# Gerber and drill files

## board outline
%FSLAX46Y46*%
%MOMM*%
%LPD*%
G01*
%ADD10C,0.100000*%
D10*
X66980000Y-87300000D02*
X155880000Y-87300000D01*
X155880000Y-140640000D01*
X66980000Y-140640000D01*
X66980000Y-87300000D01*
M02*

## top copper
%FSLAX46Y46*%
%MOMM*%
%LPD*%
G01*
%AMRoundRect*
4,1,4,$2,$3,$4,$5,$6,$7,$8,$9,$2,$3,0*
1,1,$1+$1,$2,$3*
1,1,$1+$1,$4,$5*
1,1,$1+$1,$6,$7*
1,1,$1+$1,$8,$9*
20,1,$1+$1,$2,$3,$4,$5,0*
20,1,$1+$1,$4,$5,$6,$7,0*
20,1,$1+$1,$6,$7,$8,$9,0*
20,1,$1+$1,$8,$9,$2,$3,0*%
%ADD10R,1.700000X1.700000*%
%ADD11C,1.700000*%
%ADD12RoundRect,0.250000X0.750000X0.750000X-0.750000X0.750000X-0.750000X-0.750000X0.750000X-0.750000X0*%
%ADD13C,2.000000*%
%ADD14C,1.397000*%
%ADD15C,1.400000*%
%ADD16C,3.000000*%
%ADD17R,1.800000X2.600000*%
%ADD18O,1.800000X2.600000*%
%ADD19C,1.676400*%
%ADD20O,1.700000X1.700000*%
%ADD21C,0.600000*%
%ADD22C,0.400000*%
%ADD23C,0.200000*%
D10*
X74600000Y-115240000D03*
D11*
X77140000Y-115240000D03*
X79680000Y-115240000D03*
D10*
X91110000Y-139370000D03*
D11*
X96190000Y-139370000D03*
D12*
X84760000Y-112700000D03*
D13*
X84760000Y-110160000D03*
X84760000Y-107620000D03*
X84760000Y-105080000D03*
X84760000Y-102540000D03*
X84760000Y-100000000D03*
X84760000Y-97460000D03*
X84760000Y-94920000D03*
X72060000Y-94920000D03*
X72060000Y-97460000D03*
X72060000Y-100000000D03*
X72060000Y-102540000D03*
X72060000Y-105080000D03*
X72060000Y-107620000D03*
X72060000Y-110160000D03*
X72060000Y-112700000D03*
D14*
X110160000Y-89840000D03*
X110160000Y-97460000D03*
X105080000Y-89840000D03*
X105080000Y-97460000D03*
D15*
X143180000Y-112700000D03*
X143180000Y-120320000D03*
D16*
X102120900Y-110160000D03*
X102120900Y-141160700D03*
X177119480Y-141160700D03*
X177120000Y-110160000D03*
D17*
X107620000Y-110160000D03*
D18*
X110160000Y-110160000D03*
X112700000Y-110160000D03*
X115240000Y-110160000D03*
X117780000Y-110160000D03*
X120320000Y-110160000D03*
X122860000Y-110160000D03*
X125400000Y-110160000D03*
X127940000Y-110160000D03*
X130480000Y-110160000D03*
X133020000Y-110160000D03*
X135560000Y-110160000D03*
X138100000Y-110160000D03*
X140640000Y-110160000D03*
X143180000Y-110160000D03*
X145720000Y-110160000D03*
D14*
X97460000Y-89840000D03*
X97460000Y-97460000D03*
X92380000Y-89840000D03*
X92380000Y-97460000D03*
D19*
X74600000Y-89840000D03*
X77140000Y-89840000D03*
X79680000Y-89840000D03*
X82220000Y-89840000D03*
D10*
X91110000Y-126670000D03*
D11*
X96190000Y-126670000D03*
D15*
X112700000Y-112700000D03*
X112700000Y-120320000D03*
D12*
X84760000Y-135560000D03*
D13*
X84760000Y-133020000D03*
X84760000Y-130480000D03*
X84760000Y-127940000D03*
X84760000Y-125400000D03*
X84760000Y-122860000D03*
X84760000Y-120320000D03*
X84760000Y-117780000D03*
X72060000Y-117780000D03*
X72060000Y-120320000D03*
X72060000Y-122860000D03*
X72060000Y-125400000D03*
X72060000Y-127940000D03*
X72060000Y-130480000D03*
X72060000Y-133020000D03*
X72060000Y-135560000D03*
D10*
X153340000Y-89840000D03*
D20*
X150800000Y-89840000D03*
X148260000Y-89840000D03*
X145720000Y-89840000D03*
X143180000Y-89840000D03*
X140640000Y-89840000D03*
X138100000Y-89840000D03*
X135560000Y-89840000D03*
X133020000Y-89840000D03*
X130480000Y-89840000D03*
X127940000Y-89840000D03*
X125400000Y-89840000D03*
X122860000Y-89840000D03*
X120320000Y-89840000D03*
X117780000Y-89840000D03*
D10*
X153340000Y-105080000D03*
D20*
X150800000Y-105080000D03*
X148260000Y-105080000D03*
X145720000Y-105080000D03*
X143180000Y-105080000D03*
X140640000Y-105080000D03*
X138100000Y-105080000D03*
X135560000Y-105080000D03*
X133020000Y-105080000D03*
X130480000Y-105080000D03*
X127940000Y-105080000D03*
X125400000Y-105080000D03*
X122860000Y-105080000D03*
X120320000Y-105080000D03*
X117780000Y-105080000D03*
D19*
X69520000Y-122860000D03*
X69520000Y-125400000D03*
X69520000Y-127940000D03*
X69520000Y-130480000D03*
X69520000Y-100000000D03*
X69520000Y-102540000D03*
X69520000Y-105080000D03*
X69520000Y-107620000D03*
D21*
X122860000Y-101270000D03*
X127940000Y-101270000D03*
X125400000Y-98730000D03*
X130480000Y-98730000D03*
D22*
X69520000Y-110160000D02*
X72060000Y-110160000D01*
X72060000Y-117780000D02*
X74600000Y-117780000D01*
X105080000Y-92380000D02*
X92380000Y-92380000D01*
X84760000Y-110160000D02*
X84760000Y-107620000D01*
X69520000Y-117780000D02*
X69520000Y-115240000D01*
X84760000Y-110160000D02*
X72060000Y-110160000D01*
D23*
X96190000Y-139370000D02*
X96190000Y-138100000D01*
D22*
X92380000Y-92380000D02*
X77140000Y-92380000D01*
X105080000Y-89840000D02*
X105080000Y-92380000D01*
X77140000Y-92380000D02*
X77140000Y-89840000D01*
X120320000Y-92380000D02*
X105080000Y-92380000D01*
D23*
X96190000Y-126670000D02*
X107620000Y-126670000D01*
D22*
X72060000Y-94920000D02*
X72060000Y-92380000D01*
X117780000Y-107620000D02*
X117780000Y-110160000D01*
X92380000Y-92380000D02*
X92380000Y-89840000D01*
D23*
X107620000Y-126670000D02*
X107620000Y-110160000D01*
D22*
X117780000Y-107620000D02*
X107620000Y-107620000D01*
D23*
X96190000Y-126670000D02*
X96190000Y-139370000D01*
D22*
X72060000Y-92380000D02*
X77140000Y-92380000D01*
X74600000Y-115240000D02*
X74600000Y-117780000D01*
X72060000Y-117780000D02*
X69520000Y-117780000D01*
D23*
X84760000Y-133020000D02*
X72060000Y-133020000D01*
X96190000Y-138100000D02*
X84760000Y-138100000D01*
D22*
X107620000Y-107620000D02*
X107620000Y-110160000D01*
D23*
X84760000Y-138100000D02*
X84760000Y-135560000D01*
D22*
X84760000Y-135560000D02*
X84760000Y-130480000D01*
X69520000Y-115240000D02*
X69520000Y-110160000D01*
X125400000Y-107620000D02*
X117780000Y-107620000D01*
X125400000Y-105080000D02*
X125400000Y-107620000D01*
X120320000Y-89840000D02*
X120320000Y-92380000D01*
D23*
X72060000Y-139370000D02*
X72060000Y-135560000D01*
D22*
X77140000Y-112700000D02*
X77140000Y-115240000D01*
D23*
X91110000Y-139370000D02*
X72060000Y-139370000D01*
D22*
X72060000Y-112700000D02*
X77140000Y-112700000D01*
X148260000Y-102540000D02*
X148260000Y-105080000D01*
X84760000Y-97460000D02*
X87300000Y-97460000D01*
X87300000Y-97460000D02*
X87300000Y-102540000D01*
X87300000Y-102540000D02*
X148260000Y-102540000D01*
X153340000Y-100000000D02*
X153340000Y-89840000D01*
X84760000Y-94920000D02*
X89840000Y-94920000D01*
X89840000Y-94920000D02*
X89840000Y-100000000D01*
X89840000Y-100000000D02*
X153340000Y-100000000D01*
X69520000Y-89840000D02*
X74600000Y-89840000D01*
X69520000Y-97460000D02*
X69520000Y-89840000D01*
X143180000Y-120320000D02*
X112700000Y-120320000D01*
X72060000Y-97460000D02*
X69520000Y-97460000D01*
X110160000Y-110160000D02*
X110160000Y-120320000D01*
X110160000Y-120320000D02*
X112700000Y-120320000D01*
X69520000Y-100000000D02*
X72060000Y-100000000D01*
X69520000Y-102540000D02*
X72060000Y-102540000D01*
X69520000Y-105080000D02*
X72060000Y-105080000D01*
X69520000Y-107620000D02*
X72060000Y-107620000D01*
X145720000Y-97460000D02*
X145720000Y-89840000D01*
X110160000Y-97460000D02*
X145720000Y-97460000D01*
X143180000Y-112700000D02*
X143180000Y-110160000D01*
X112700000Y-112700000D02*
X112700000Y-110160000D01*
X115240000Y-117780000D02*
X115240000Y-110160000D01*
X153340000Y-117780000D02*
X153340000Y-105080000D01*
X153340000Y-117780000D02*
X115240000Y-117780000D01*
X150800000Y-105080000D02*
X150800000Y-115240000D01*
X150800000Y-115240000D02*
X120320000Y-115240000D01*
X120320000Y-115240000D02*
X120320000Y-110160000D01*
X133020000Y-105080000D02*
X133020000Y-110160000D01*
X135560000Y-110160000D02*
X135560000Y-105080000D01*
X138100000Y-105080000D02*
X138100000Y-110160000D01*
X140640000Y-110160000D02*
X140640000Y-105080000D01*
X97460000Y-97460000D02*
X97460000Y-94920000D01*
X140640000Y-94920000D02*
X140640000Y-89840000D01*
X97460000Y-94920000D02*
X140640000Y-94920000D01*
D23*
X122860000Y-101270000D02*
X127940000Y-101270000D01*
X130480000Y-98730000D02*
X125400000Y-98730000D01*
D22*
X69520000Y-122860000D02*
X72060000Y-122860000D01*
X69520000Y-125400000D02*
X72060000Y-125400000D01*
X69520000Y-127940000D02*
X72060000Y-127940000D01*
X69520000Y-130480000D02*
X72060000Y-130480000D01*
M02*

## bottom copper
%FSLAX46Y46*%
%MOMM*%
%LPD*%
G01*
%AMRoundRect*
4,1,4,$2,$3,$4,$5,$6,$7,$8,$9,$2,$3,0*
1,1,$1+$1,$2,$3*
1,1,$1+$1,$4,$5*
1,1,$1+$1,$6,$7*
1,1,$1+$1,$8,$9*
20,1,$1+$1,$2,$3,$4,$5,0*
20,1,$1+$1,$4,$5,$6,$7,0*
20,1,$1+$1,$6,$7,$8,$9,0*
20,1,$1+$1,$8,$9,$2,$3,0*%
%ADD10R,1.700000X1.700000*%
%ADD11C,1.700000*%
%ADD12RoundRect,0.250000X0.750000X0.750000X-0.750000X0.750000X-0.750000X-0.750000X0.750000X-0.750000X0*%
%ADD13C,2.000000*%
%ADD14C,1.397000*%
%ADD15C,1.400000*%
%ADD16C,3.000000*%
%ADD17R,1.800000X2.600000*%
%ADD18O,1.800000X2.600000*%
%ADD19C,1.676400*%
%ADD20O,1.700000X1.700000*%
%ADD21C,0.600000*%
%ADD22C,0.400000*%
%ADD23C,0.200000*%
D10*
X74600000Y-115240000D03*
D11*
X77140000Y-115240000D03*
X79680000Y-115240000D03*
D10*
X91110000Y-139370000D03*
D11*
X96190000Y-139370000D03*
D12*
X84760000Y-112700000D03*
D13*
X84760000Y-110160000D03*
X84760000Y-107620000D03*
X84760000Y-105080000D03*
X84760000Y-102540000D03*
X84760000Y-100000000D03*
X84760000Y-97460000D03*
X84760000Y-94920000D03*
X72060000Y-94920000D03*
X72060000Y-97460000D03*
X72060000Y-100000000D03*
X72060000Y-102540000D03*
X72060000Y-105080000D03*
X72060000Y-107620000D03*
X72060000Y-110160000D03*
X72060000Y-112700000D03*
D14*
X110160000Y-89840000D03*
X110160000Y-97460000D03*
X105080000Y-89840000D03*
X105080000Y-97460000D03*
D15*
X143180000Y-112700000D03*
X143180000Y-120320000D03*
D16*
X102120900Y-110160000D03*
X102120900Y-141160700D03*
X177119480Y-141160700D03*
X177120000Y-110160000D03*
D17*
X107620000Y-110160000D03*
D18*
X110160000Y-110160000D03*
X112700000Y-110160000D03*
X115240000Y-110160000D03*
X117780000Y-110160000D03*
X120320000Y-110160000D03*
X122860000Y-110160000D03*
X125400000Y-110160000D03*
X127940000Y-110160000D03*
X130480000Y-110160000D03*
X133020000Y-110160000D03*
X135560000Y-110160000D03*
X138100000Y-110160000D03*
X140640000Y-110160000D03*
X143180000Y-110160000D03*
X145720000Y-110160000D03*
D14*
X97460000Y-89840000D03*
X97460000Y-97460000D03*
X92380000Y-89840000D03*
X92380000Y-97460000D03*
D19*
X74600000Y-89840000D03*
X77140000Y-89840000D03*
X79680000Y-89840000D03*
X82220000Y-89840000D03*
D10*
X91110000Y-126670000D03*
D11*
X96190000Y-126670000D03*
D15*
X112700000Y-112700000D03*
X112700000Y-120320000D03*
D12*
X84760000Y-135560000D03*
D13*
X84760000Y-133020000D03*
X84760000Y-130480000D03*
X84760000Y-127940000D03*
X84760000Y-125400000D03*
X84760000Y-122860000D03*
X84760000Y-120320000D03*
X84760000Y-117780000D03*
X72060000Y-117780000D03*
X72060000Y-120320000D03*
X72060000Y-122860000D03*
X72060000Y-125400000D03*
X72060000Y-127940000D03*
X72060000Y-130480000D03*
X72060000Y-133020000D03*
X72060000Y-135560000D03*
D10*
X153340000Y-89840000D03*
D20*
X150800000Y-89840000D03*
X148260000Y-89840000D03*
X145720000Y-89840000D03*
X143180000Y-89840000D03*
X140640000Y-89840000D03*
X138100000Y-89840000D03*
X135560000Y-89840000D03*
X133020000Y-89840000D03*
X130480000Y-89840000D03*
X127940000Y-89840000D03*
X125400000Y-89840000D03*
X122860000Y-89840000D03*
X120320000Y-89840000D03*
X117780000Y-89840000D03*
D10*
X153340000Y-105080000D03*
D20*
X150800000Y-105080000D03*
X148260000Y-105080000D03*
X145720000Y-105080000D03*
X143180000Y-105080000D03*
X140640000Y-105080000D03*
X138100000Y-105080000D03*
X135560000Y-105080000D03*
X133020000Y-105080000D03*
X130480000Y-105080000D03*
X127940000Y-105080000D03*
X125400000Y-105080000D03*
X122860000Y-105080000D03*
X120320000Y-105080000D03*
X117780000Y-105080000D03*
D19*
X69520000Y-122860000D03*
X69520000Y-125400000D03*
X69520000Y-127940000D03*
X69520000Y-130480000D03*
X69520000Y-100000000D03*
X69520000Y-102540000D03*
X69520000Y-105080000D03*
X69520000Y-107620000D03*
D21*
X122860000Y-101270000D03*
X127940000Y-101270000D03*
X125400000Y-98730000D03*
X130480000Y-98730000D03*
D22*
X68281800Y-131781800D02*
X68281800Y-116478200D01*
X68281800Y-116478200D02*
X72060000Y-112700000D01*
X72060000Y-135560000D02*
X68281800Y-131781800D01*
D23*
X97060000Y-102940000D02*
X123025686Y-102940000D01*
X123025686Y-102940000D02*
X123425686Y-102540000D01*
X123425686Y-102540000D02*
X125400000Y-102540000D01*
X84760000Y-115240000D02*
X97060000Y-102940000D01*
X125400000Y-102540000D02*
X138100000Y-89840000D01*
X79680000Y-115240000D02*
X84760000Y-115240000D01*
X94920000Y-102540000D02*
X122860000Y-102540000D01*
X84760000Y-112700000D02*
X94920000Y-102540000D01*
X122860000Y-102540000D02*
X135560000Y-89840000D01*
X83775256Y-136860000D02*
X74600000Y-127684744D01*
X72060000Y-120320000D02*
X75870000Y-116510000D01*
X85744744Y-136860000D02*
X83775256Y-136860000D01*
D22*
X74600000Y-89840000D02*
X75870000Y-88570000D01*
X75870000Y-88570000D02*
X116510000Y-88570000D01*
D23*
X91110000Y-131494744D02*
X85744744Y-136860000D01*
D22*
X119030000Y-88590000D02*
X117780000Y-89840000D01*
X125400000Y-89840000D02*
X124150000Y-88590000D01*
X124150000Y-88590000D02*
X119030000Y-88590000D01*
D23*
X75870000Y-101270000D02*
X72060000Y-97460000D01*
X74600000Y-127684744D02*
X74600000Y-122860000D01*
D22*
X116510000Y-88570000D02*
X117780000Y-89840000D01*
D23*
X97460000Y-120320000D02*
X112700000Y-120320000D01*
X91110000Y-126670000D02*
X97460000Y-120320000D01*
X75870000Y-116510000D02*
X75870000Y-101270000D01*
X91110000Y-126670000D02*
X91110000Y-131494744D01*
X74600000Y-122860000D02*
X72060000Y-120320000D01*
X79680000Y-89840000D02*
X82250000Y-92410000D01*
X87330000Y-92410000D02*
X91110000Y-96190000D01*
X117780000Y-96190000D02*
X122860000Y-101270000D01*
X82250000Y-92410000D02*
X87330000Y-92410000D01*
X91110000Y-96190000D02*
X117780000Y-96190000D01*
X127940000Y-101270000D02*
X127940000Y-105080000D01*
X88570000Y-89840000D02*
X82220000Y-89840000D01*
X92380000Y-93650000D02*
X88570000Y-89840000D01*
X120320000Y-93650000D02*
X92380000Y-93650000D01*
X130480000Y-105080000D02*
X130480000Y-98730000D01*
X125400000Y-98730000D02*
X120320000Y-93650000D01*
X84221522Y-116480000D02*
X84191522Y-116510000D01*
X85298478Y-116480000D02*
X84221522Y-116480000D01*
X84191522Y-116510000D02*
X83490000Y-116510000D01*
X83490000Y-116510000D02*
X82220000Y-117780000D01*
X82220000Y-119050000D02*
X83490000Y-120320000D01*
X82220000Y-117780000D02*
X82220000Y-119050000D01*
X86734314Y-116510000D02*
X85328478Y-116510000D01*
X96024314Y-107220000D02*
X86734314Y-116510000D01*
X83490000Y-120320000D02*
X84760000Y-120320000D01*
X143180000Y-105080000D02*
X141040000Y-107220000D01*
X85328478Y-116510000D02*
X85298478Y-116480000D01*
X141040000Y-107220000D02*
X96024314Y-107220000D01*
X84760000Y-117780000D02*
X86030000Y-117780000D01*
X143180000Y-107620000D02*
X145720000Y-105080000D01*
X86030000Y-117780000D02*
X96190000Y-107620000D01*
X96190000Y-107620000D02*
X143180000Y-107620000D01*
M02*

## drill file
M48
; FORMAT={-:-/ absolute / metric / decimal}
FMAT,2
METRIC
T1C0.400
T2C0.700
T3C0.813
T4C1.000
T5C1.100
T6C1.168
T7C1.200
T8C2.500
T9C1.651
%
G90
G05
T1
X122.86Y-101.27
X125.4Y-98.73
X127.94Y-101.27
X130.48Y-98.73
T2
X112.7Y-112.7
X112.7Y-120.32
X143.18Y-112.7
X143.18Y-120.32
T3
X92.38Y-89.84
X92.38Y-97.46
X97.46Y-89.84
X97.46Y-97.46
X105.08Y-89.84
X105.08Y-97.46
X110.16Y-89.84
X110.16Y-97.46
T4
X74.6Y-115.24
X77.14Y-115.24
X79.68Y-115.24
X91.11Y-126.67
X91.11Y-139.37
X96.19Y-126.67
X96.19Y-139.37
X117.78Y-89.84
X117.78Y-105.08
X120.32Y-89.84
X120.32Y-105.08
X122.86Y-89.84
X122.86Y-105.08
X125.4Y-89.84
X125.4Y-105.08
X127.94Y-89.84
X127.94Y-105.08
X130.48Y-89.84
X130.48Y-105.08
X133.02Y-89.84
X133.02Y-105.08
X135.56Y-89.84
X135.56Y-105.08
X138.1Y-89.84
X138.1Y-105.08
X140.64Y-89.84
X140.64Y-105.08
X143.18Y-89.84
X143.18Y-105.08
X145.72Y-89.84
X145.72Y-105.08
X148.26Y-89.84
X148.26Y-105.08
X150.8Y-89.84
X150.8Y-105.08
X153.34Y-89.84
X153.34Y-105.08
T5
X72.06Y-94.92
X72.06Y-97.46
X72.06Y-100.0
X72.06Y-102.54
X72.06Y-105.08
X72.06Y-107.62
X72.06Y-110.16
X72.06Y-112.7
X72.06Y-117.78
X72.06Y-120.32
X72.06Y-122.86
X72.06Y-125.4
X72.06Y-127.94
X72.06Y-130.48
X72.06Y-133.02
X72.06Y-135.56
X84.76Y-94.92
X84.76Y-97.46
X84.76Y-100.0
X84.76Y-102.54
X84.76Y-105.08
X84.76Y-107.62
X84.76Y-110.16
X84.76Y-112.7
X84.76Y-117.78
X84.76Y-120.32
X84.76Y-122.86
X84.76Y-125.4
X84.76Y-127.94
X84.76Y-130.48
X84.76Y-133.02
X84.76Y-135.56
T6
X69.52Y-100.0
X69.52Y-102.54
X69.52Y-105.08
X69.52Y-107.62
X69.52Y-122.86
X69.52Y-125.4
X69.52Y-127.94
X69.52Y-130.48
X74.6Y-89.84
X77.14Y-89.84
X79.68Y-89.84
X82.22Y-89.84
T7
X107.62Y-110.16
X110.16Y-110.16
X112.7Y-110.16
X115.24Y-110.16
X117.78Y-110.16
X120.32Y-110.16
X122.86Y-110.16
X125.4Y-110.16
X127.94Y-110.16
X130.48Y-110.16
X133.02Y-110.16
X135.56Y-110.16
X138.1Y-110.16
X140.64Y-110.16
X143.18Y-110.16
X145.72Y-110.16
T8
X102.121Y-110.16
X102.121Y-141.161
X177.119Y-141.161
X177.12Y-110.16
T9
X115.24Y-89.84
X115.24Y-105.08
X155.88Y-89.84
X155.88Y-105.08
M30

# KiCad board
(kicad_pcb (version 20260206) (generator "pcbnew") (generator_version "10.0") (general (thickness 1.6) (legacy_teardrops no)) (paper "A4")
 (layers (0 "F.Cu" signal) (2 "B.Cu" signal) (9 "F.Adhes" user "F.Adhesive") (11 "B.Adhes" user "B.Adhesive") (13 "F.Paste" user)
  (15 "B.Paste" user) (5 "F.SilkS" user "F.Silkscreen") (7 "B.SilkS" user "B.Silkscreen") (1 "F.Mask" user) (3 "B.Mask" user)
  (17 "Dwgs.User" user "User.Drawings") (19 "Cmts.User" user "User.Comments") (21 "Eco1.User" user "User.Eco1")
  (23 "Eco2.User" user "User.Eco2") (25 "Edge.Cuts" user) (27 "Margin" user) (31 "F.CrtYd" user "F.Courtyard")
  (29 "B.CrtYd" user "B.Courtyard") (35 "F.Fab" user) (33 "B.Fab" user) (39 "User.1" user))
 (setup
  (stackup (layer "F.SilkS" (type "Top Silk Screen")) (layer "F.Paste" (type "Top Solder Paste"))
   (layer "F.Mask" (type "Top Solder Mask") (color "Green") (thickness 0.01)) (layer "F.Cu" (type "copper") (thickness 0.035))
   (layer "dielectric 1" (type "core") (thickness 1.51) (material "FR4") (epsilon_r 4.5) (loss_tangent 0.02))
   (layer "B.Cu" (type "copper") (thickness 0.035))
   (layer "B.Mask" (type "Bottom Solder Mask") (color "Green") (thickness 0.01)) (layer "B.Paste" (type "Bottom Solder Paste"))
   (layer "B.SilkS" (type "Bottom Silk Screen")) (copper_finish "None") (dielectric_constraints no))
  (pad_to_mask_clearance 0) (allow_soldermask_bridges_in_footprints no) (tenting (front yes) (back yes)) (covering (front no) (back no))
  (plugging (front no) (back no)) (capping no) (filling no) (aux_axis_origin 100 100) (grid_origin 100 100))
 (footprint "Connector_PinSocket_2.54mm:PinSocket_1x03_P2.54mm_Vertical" (layer "F.Cu") (at 74.6 115.24 90)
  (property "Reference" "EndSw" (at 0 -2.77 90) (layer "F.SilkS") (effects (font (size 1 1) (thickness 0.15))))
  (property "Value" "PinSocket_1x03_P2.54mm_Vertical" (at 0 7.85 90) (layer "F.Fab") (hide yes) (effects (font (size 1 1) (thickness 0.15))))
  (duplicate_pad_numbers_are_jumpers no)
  (pad "1" thru_hole rect (at 0 0 90) (size 1.7 1.7) (drill 1) (layers "*.Cu" "*.Mask") (remove_unused_layers no) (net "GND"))
  (pad "2" thru_hole circle (at 0 2.54 90) (size 1.7 1.7) (drill 1) (layers "*.Cu" "*.Mask") (remove_unused_layers no) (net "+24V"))
  (pad "3" thru_hole circle (at 0 5.08 90) (size 1.7 1.7) (drill 1) (layers "*.Cu" "*.Mask") (remove_unused_layers no) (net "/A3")))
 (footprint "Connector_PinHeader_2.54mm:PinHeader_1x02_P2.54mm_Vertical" (layer "F.Cu") (at 91.11 139.37 90)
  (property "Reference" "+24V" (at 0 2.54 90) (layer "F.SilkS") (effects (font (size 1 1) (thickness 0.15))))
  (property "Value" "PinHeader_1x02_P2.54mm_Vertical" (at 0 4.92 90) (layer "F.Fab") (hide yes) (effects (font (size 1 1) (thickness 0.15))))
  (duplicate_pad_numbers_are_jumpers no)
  (pad "1" thru_hole rect (at 0 0 90) (size 1.7 1.7) (drill 1) (layers "*.Cu" "*.Mask") (remove_unused_layers no) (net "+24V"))
  (pad "2" thru_hole circle (at 0 5.08 90) (size 1.7 1.7) (drill 1) (layers "*.Cu" "*.Mask") (remove_unused_layers no) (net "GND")))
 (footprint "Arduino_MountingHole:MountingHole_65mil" (layer "F.Cu") (at 155.88 105.08 180)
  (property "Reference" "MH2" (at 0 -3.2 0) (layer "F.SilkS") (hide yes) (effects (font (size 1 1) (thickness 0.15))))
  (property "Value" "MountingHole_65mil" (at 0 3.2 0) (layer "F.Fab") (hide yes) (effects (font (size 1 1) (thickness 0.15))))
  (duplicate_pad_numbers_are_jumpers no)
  (pad "" np_thru_hole circle (at 0 0 180) (size 1.651 1.651) (drill 1.651) (layers "*.Cu" "*.Mask")))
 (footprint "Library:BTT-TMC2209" (layer "F.Cu") (at 86.03 113.97 180)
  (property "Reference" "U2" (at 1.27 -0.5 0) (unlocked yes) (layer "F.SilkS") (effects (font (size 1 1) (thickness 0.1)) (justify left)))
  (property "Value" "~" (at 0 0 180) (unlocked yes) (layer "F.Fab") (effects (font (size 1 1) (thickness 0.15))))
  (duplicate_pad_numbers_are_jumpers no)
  (pad "1" thru_hole roundrect (at 1.27 1.27 180) (size 2 2) (drill 1.1) (layers "*.Cu" "*.Mask") (remove_unused_layers no)
   (roundrect_rratio 0.125) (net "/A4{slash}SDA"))
  (pad "2" thru_hole circle (at 1.27 3.81 180) (size 2 2) (drill 1.1) (layers "*.Cu" "*.Mask") (remove_unused_layers no) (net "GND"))
  (pad "3" thru_hole circle (at 1.27 6.35 180) (size 2 2) (drill 1.1) (layers "*.Cu" "*.Mask") (remove_unused_layers no) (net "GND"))
  (pad "4" thru_hole circle (at 1.27 8.89 180) (size 2 2) (drill 1.1) (layers "*.Cu" "*.Mask") (remove_unused_layers no)
   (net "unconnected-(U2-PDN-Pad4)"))
  (pad "5" thru_hole circle (at 1.27 11.43 180) (size 2 2) (drill 1.1) (layers "*.Cu" "*.Mask") (remove_unused_layers no)
   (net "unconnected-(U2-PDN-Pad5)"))
  (pad "6" thru_hole circle (at 1.27 13.97 180) (size 2 2) (drill 1.1) (layers "*.Cu" "*.Mask") (remove_unused_layers no)
   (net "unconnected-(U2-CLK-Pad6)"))
  (pad "7" thru_hole circle (at 1.27 16.51 180) (size 2 2) (drill 1.1) (layers "*.Cu" "*.Mask") (remove_unused_layers no)
   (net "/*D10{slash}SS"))
  (pad "8" thru_hole circle (at 1.27 19.05 180) (size 2 2) (drill 1.1) (layers "*.Cu" "*.Mask") (remove_unused_layers no)
   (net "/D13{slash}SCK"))
  (pad "9" thru_hole circle (at 13.97 19.05 180) (size 2 2) (drill 1.1) (layers "*.Cu" "*.Mask") (remove_unused_layers no) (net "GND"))
  (pad "10" thru_hole circle (at 13.97 16.51 180) (size 2 2) (drill 1.1) (layers "*.Cu" "*.Mask") (remove_unused_layers no) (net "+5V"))
  (pad "11" thru_hole circle (at 13.97 13.97 180) (size 2 2) (drill 1.1) (layers "*.Cu" "*.Mask") (remove_unused_layers no)
   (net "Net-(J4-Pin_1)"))
  (pad "12" thru_hole circle (at 13.97 11.43 180) (size 2 2) (drill 1.1) (layers "*.Cu" "*.Mask") (remove_unused_layers no)
   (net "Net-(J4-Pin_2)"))
  (pad "13" thru_hole circle (at 13.97 8.89 180) (size 2 2) (drill 1.1) (layers "*.Cu" "*.Mask") (remove_unused_layers no)
   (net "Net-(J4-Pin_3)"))
  (pad "14" thru_hole circle (at 13.97 6.35 180) (size 2 2) (drill 1.1) (layers "*.Cu" "*.Mask") (remove_unused_layers no)
   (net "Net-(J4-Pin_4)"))
  (pad "15" thru_hole circle (at 13.97 3.81 180) (size 2 2) (drill 1.1) (layers "*.Cu" "*.Mask") (remove_unused_layers no) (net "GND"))
  (pad "16" thru_hole circle (at 13.97 1.27 180) (size 2 2) (drill 1.1) (layers "*.Cu" "*.Mask") (remove_unused_layers no) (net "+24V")))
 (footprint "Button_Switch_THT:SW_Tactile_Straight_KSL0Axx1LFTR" (layer "F.Cu") (at 110.16 89.84 -90)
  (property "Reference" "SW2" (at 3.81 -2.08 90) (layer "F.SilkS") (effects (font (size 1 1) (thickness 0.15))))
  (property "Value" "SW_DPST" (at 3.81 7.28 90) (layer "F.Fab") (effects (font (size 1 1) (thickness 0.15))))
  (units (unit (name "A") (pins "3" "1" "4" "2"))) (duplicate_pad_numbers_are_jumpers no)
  (pad "1" thru_hole circle (at 0 0 270) (size 1.397 1.397) (drill 0.8128) (layers "*.Cu" "*.Mask") (remove_unused_layers no))
  (pad "1" thru_hole circle (at 7.62 0 270) (size 1.397 1.397) (drill 0.8128) (layers "*.Cu" "*.Mask") (remove_unused_layers no) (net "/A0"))
  (pad "2" thru_hole circle (at 0 5.08 270) (size 1.397 1.397) (drill 0.8128) (layers "*.Cu" "*.Mask") (remove_unused_layers no) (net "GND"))
  (pad "2" thru_hole circle (at 7.62 5.08 270) (size 1.397 1.397) (drill 0.8128) (layers "*.Cu" "*.Mask") (remove_unused_layers no)))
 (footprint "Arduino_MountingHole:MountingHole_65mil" (layer "F.Cu") (at 115.24 89.84 180)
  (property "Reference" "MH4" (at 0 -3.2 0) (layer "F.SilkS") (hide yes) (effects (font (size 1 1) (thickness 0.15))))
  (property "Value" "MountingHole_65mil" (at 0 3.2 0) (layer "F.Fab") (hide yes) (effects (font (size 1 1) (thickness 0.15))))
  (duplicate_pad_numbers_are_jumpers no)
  (pad "" np_thru_hole circle (at 0 0 180) (size 1.651 1.651) (drill 1.651) (layers "*.Cu" "*.Mask")))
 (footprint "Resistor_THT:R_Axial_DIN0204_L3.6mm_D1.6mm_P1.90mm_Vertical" (layer "F.Cu") (at 143.18 112.7 -90)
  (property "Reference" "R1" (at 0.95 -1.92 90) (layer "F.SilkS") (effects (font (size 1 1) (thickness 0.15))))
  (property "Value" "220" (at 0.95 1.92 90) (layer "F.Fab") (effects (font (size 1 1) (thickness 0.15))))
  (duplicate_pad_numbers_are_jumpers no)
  (pad "1" thru_hole circle (at 0 0 270) (size 1.4 1.4) (drill 0.7) (layers "*.Cu" "*.Mask") (remove_unused_layers no)
   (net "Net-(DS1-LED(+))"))
  (pad "2" thru_hole circle (at 7.62 0 270) (size 1.4 1.4) (drill 0.7) (layers "*.Cu" "*.Mask") (remove_unused_layers no) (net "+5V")))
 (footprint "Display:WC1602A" (layer "F.Cu") (at 107.62 110.16)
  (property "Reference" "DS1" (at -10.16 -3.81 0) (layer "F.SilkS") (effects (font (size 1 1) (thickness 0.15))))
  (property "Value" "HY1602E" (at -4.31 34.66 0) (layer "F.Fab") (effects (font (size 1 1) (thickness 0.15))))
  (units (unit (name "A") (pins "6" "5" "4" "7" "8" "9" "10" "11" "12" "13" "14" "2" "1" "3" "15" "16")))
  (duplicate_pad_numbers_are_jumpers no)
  (pad "" thru_hole circle (at -5.4991 0) (size 3 3) (drill 2.5) (layers "*.Cu" "*.Mask") (remove_unused_layers no))
  (pad "" thru_hole circle (at -5.4991 31.0007) (size 3 3) (drill 2.5) (layers "*.Cu" "Dwgs.User") (remove_unused_layers no))
  (pad "" thru_hole circle (at 69.49948 31.0007) (size 3 3) (drill 2.5) (layers "*.Cu" "*.Mask") (remove_unused_layers no))
  (pad "" thru_hole circle (at 69.5 0) (size 3 3) (drill 2.5) (layers "*.Cu" "*.Mask" "Dwgs.User") (remove_unused_layers no))
  (pad "1" thru_hole rect (at 0 0) (size 1.8 2.6) (drill 1.2) (layers "*.Cu" "*.Mask") (remove_unused_layers no) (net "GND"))
  (pad "2" thru_hole oval (at 2.54 0) (size 1.8 2.6) (drill 1.2) (layers "*.Cu" "*.Mask") (remove_unused_layers no) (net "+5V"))
  (pad "3" thru_hole oval (at 5.08 0) (size 1.8 2.6) (drill 1.2) (layers "*.Cu" "*.Mask") (remove_unused_layers no) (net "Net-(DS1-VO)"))
  (pad "4" thru_hole oval (at 7.62 0) (size 1.8 2.6) (drill 1.2) (layers "*.Cu" "*.Mask") (remove_unused_layers no) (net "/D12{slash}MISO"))
  (pad "5" thru_hole oval (at 10.16 0) (size 1.8 2.6) (drill 1.2) (layers "*.Cu" "*.Mask") (remove_unused_layers no) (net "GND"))
  (pad "6" thru_hole oval (at 12.7 0) (size 1.8 2.6) (drill 1.2) (layers "*.Cu" "*.Mask") (remove_unused_layers no) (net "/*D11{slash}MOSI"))
  (pad "7" thru_hole oval (at 15.24 0) (size 1.8 2.6) (drill 1.2) (layers "*.Cu" "*.Mask") (remove_unused_layers no)
   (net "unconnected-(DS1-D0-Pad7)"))
  (pad "8" thru_hole oval (at 17.78 0) (size 1.8 2.6) (drill 1.2) (layers "*.Cu" "*.Mask") (remove_unused_layers no)
   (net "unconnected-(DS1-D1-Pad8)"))
  (pad "9" thru_hole oval (at 20.32 0) (size 1.8 2.6) (drill 1.2) (layers "*.Cu" "*.Mask") (remove_unused_layers no)
   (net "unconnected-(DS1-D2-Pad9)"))
  (pad "10" thru_hole oval (at 22.86 0) (size 1.8 2.6) (drill 1.2) (layers "*.Cu" "*.Mask") (remove_unused_layers no)
   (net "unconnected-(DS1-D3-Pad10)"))
  (pad "11" thru_hole oval (at 25.4 0) (size 1.8 2.6) (drill 1.2) (layers "*.Cu" "*.Mask") (remove_unused_layers no) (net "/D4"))
  (pad "12" thru_hole oval (at 27.94 0) (size 1.8 2.6) (drill 1.2) (layers "*.Cu" "*.Mask") (remove_unused_layers no) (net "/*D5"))
  (pad "13" thru_hole oval (at 30.48 0) (size 1.8 2.6) (drill 1.2) (layers "*.Cu" "*.Mask") (remove_unused_layers no) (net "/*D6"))
  (pad "14" thru_hole oval (at 33.02 0) (size 1.8 2.6) (drill 1.2) (layers "*.Cu" "*.Mask") (remove_unused_layers no) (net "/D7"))
  (pad "15" thru_hole oval (at 35.56 0) (size 1.8 2.6) (drill 1.2) (layers "*.Cu" "*.Mask") (remove_unused_layers no)
   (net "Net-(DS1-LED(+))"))
  (pad "16" thru_hole oval (at 38.1 0) (size 1.8 2.6) (drill 1.2) (layers "*.Cu" "*.Mask") (remove_unused_layers no) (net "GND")))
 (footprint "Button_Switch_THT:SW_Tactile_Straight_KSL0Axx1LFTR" (layer "F.Cu") (at 97.46 89.84 -90)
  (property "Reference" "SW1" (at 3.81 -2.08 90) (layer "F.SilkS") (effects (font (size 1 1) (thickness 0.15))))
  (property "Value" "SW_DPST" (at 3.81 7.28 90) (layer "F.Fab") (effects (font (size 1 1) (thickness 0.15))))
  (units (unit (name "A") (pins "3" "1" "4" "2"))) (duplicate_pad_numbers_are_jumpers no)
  (pad "1" thru_hole circle (at 0 0 270) (size 1.397 1.397) (drill 0.8128) (layers "*.Cu" "*.Mask") (remove_unused_layers no))
  (pad "1" thru_hole circle (at 7.62 0 270) (size 1.397 1.397) (drill 0.8128) (layers "*.Cu" "*.Mask") (remove_unused_layers no) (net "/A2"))
  (pad "2" thru_hole circle (at 0 5.08 270) (size 1.397 1.397) (drill 0.8128) (layers "*.Cu" "*.Mask") (remove_unused_layers no) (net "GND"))
  (pad "2" thru_hole circle (at 7.62 5.08 270) (size 1.397 1.397) (drill 0.8128) (layers "*.Cu" "*.Mask") (remove_unused_layers no)))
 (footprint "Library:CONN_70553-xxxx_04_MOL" (layer "F.Cu") (at 74.6 89.84 180)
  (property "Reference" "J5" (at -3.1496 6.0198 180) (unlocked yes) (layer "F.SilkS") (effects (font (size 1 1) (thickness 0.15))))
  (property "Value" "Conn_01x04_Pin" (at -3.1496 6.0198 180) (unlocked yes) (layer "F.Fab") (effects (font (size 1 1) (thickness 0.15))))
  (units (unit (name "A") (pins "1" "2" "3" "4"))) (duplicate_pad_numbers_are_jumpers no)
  (pad "1" thru_hole circle (at 0 0 180) (size 1.6764 1.6764) (drill 1.1684) (layers "*.Cu" "*.Mask") (remove_unused_layers no) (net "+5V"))
  (pad "2" thru_hole circle (at -2.54 0 180) (size 1.6764 1.6764) (drill 1.1684) (layers "*.Cu" "*.Mask") (remove_unused_layers no)
   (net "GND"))
  (pad "3" thru_hole circle (at -5.08 0 180) (size 1.6764 1.6764) (drill 1.1684) (layers "*.Cu" "*.Mask") (remove_unused_layers no)
   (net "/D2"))
  (pad "4" thru_hole circle (at -7.62 0 180) (size 1.6764 1.6764) (drill 1.1684) (layers "*.Cu" "*.Mask") (remove_unused_layers no)
   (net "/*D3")))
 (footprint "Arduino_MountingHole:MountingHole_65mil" (layer "F.Cu") (at 155.88 89.84 180)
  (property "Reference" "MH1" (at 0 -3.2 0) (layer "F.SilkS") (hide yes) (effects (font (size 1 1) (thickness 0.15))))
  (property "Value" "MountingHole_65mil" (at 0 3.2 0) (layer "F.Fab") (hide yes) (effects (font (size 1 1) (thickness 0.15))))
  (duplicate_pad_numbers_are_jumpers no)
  (pad "" np_thru_hole circle (at 0 0 180) (size 1.651 1.651) (drill 1.651) (layers "*.Cu" "*.Mask")))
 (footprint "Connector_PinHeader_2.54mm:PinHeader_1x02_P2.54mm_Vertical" (layer "F.Cu") (at 91.11 126.67 90)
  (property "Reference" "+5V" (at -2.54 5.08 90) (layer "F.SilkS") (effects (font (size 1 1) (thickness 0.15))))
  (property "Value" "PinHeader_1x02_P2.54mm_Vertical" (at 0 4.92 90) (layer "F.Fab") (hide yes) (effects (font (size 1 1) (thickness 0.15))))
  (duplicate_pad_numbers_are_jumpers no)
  (pad "1" thru_hole rect (at 0 0 90) (size 1.7 1.7) (drill 1) (layers "*.Cu" "*.Mask") (remove_unused_layers no) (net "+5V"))
  (pad "2" thru_hole circle (at 0 5.08 90) (size 1.7 1.7) (drill 1) (layers "*.Cu" "*.Mask") (remove_unused_layers no) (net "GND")))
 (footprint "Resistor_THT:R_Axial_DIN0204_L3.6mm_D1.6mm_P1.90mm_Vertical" (layer "F.Cu") (at 112.7 112.7 -90)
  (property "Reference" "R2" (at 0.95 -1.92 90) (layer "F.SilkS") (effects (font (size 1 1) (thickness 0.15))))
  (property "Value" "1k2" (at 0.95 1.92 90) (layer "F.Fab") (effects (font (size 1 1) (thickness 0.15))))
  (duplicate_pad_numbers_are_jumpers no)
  (pad "1" thru_hole circle (at 0 0 270) (size 1.4 1.4) (drill 0.7) (layers "*.Cu" "*.Mask") (remove_unused_layers no) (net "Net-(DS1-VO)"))
  (pad "2" thru_hole circle (at 7.62 0 270) (size 1.4 1.4) (drill 0.7) (layers "*.Cu" "*.Mask") (remove_unused_layers no) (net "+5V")))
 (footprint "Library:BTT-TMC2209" (layer "F.Cu") (at 86.03 136.83 180)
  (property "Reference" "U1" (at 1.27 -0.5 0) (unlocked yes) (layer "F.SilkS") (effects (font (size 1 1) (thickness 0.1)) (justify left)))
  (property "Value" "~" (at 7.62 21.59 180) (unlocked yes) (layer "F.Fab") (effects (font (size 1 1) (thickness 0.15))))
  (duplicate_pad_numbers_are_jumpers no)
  (pad "1" thru_hole roundrect (at 1.27 1.27 180) (size 2 2) (drill 1.1) (layers "*.Cu" "*.Mask") (remove_unused_layers no)
   (roundrect_rratio 0.125) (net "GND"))
  (pad "2" thru_hole circle (at 1.27 3.81 180) (size 2 2) (drill 1.1) (layers "*.Cu" "*.Mask") (remove_unused_layers no) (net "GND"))
  (pad "3" thru_hole circle (at 1.27 6.35 180) (size 2 2) (drill 1.1) (layers "*.Cu" "*.Mask") (remove_unused_layers no) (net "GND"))
  (pad "4" thru_hole circle (at 1.27 8.89 180) (size 2 2) (drill 1.1) (layers "*.Cu" "*.Mask") (remove_unused_layers no)
   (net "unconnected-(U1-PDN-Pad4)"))
  (pad "5" thru_hole circle (at 1.27 11.43 180) (size 2 2) (drill 1.1) (layers "*.Cu" "*.Mask") (remove_unused_layers no)
   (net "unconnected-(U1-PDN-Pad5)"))
  (pad "6" thru_hole circle (at 1.27 13.97 180) (size 2 2) (drill 1.1) (layers "*.Cu" "*.Mask") (remove_unused_layers no)
   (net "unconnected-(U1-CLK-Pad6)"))
  (pad "7" thru_hole circle (at 1.27 16.51 180) (size 2 2) (drill 1.1) (layers "*.Cu" "*.Mask") (remove_unused_layers no) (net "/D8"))
  (pad "8" thru_hole circle (at 1.27 19.05 180) (size 2 2) (drill 1.1) (layers "*.Cu" "*.Mask") (remove_unused_layers no) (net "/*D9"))
  (pad "9" thru_hole circle (at 13.97 19.05 180) (size 2 2) (drill 1.1) (layers "*.Cu" "*.Mask") (remove_unused_layers no) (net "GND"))
  (pad "10" thru_hole circle (at 13.97 16.51 180) (size 2 2) (drill 1.1) (layers "*.Cu" "*.Mask") (remove_unused_layers no) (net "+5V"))
  (pad "11" thru_hole circle (at 13.97 13.97 180) (size 2 2) (drill 1.1) (layers "*.Cu" "*.Mask") (remove_unused_layers no)
   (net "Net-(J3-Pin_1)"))
  (pad "12" thru_hole circle (at 13.97 11.43 180) (size 2 2) (drill 1.1) (layers "*.Cu" "*.Mask") (remove_unused_layers no)
   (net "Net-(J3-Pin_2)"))
  (pad "13" thru_hole circle (at 13.97 8.89 180) (size 2 2) (drill 1.1) (layers "*.Cu" "*.Mask") (remove_unused_layers no)
   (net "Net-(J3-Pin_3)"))
  (pad "14" thru_hole circle (at 13.97 6.35 180) (size 2 2) (drill 1.1) (layers "*.Cu" "*.Mask") (remove_unused_layers no)
   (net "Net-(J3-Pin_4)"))
  (pad "15" thru_hole circle (at 13.97 3.81 180) (size 2 2) (drill 1.1) (layers "*.Cu" "*.Mask") (remove_unused_layers no) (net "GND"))
  (pad "16" thru_hole circle (at 13.97 1.27 180) (size 2 2) (drill 1.1) (layers "*.Cu" "*.Mask") (remove_unused_layers no) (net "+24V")))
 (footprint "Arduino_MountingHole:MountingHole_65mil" (layer "F.Cu") (at 115.24 105.08 180)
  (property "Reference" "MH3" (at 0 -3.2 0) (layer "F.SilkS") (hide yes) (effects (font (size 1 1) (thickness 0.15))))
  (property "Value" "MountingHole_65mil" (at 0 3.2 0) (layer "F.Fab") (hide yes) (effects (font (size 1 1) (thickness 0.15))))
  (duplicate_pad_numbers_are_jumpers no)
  (pad "" np_thru_hole circle (at 0 0 180) (size 1.651 1.651) (drill 1.651) (layers "*.Cu" "*.Mask")))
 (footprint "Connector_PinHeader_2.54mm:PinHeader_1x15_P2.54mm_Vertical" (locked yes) (layer "B.Cu") (at 153.34 89.84 90)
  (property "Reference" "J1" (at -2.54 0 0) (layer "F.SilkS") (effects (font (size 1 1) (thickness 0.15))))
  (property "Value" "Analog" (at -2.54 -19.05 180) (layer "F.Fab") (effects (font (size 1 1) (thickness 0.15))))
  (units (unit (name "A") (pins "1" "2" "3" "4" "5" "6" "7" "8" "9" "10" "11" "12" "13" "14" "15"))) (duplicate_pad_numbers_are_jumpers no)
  (pad "1" thru_hole rect (at 0 0 90) (size 1.7 1.7) (drill 1) (layers "*.Cu" "*.Mask") (remove_unused_layers no) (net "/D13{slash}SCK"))
  (pad "2" thru_hole oval (at 0 -2.54 90) (size 1.7 1.7) (drill 1) (layers "*.Cu" "*.Mask") (remove_unused_layers no) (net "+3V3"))
  (pad "3" thru_hole oval (at 0 -5.08 90) (size 1.7 1.7) (drill 1) (layers "*.Cu" "*.Mask") (remove_unused_layers no) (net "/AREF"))
  (pad "4" thru_hole oval (at 0 -7.62 90) (size 1.7 1.7) (drill 1) (layers "*.Cu" "*.Mask") (remove_unused_layers no) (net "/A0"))
  (pad "5" thru_hole oval (at 0 -10.16 90) (size 1.7 1.7) (drill 1) (layers "*.Cu" "*.Mask") (remove_unused_layers no) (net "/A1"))
  (pad "6" thru_hole oval (at 0 -12.7 90) (size 1.7 1.7) (drill 1) (layers "*.Cu" "*.Mask") (remove_unused_layers no) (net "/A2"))
  (pad "7" thru_hole oval (at 0 -15.24 90) (size 1.7 1.7) (drill 1) (layers "*.Cu" "*.Mask") (remove_unused_layers no) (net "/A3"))
  (pad "8" thru_hole oval (at 0 -17.78 90) (size 1.7 1.7) (drill 1) (layers "*.Cu" "*.Mask") (remove_unused_layers no) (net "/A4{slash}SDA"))
  (pad "9" thru_hole oval (at 0 -20.32 90) (size 1.7 1.7) (drill 1) (layers "*.Cu" "*.Mask") (remove_unused_layers no) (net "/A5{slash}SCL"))
  (pad "10" thru_hole oval (at 0 -22.86 90) (size 1.7 1.7) (drill 1) (layers "*.Cu" "*.Mask") (remove_unused_layers no) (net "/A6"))
  (pad "11" thru_hole oval (at 0 -25.4 90) (size 1.7 1.7) (drill 1) (layers "*.Cu" "*.Mask") (remove_unused_layers no) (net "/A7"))
  (pad "12" thru_hole oval (at 0 -27.94 90) (size 1.7 1.7) (drill 1) (layers "*.Cu" "*.Mask") (remove_unused_layers no) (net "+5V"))
  (pad "13" thru_hole oval (at 0 -30.48 90) (size 1.7 1.7) (drill 1) (layers "*.Cu" "*.Mask") (remove_unused_layers no) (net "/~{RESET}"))
  (pad "14" thru_hole oval (at 0 -33.02 90) (size 1.7 1.7) (drill 1) (layers "*.Cu" "*.Mask") (remove_unused_layers no) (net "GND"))
  (pad "15" thru_hole oval (at 0 -35.56 90) (size 1.7 1.7) (drill 1) (layers "*.Cu" "*.Mask") (remove_unused_layers no) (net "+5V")))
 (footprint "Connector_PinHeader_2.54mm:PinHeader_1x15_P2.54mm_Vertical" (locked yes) (layer "B.Cu") (at 153.34 105.08 90)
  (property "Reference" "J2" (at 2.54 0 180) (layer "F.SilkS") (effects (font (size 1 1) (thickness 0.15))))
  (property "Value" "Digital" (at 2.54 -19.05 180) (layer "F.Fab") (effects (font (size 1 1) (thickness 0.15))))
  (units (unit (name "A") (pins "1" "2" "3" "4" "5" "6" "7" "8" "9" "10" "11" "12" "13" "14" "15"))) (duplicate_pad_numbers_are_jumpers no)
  (pad "1" thru_hole rect (at 0 0 90) (size 1.7 1.7) (drill 1) (layers "*.Cu" "*.Mask") (remove_unused_layers no) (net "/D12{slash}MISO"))
  (pad "2" thru_hole oval (at 0 -2.54 90) (size 1.7 1.7) (drill 1) (layers "*.Cu" "*.Mask") (remove_unused_layers no)
   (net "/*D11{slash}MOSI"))
  (pad "3" thru_hole oval (at 0 -5.08 90) (size 1.7 1.7) (drill 1) (layers "*.Cu" "*.Mask") (remove_unused_layers no) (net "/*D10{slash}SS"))
  (pad "4" thru_hole oval (at 0 -7.62 90) (size 1.7 1.7) (drill 1) (layers "*.Cu" "*.Mask") (remove_unused_layers no) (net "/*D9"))
  (pad "5" thru_hole oval (at 0 -10.16 90) (size 1.7 1.7) (drill 1) (layers "*.Cu" "*.Mask") (remove_unused_layers no) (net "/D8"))
  (pad "6" thru_hole oval (at 0 -12.7 90) (size 1.7 1.7) (drill 1) (layers "*.Cu" "*.Mask") (remove_unused_layers no) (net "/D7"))
  (pad "7" thru_hole oval (at 0 -15.24 90) (size 1.7 1.7) (drill 1) (layers "*.Cu" "*.Mask") (remove_unused_layers no) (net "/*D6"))
  (pad "8" thru_hole oval (at 0 -17.78 90) (size 1.7 1.7) (drill 1) (layers "*.Cu" "*.Mask") (remove_unused_layers no) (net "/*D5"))
  (pad "9" thru_hole oval (at 0 -20.32 90) (size 1.7 1.7) (drill 1) (layers "*.Cu" "*.Mask") (remove_unused_layers no) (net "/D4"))
  (pad "10" thru_hole oval (at 0 -22.86 90) (size 1.7 1.7) (drill 1) (layers "*.Cu" "*.Mask") (remove_unused_layers no) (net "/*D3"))
  (pad "11" thru_hole oval (at 0 -25.4 90) (size 1.7 1.7) (drill 1) (layers "*.Cu" "*.Mask") (remove_unused_layers no) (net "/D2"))
  (pad "12" thru_hole oval (at 0 -27.94 90) (size 1.7 1.7) (drill 1) (layers "*.Cu" "*.Mask") (remove_unused_layers no) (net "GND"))
  (pad "13" thru_hole oval (at 0 -30.48 90) (size 1.7 1.7) (drill 1) (layers "*.Cu" "*.Mask") (remove_unused_layers no) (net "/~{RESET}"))
  (pad "14" thru_hole oval (at 0 -33.02 90) (size 1.7 1.7) (drill 1) (layers "*.Cu" "*.Mask") (remove_unused_layers no) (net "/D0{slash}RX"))
  (pad "15" thru_hole oval (at 0 -35.56 90) (size 1.7 1.7) (drill 1) (layers "*.Cu" "*.Mask") (remove_unused_layers no) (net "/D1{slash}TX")))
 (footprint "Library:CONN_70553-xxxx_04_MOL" (layer "B.Cu") (at 69.52 122.86 90)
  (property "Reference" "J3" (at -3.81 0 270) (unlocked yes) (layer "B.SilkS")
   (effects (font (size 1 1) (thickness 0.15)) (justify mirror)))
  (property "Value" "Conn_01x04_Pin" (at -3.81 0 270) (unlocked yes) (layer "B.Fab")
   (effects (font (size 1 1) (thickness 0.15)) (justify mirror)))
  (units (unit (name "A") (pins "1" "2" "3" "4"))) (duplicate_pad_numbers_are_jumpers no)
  (pad "1" thru_hole circle (at 0 0 90) (size 1.6764 1.6764) (drill 1.1684) (layers "*.Cu" "*.Mask") (remove_unused_layers no)
   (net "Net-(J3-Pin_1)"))
  (pad "2" thru_hole circle (at -2.54 0 90) (size 1.6764 1.6764) (drill 1.1684) (layers "*.Cu" "*.Mask") (remove_unused_layers no)
   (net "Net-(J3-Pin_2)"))
  (pad "3" thru_hole circle (at -5.08 0 90) (size 1.6764 1.6764) (drill 1.1684) (layers "*.Cu" "*.Mask") (remove_unused_layers no)
   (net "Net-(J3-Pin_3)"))
  (pad "4" thru_hole circle (at -7.62 0 90) (size 1.6764 1.6764) (drill 1.1684) (layers "*.Cu" "*.Mask") (remove_unused_layers no)
   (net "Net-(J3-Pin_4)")))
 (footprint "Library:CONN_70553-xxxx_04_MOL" (layer "B.Cu") (at 69.52 100 90)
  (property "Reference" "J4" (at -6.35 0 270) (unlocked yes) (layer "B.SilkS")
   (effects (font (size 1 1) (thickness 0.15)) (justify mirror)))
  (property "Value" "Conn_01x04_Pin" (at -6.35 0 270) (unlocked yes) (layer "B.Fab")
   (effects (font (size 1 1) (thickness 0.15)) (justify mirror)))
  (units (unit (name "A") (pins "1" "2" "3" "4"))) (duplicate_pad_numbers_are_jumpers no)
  (pad "1" thru_hole circle (at 0 0 90) (size 1.6764 1.6764) (drill 1.1684) (layers "*.Cu" "*.Mask") (remove_unused_layers no)
   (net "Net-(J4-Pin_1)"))
  (pad "2" thru_hole circle (at -2.54 0 90) (size 1.6764 1.6764) (drill 1.1684) (layers "*.Cu" "*.Mask") (remove_unused_layers no)
   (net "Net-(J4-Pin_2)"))
  (pad "3" thru_hole circle (at -5.08 0 90) (size 1.6764 1.6764) (drill 1.1684) (layers "*.Cu" "*.Mask") (remove_unused_layers no)
   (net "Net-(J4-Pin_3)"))
  (pad "4" thru_hole circle (at -7.62 0 90) (size 1.6764 1.6764) (drill 1.1684) (layers "*.Cu" "*.Mask") (remove_unused_layers no)
   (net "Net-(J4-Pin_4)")))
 (gr_rect (start 66.98 87.3) (end 155.88 140.64) (stroke (width 0.1) (type solid)) (fill no) (layer "Edge.Cuts"))
 (segment (start 69.52 110.16) (end 72.06 110.16) (width 0.4) (layer "F.Cu") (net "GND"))
 (segment (start 72.06 117.78) (end 74.6 117.78) (width 0.4) (layer "F.Cu") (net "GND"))
 (segment (start 105.08 92.38) (end 92.38 92.38) (width 0.4) (layer "F.Cu") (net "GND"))
 (segment (start 84.76 110.16) (end 84.76 107.62) (width 0.4) (layer "F.Cu") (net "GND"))
 (segment (start 69.52 117.78) (end 69.52 115.24) (width 0.4) (layer "F.Cu") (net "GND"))
 (segment (start 84.76 110.16) (end 72.06 110.16) (width 0.4) (layer "F.Cu") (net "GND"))
 (segment (start 96.19 139.37) (end 96.19 138.1) (width 0.2) (layer "F.Cu") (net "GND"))
 (segment (start 92.38 92.38) (end 77.14 92.38) (width 0.4) (layer "F.Cu") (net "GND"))
 (segment (start 105.08 89.84) (end 105.08 92.38) (width 0.4) (layer "F.Cu") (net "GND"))
 (segment (start 77.14 92.38) (end 77.14 89.84) (width 0.4) (layer "F.Cu") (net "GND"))
 (segment (start 120.32 92.38) (end 105.08 92.38) (width 0.4) (layer "F.Cu") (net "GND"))
 (segment (start 96.19 126.67) (end 107.62 126.67) (width 0.2) (layer "F.Cu") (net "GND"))
 (segment (start 72.06 94.92) (end 72.06 92.38) (width 0.4) (layer "F.Cu") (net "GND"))
 (segment (start 117.78 107.62) (end 117.78 110.16) (width 0.4) (layer "F.Cu") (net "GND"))
 (segment (start 92.38 92.38) (end 92.38 89.84) (width 0.4) (layer "F.Cu") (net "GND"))
 (segment (start 107.62 126.67) (end 107.62 110.16) (width 0.2) (layer "F.Cu") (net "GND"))
 (segment (start 117.78 107.62) (end 107.62 107.62) (width 0.4) (layer "F.Cu") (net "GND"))
 (segment (start 96.19 126.67) (end 96.19 139.37) (width 0.2) (layer "F.Cu") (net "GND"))
 (segment (start 72.06 92.38) (end 77.14 92.38) (width 0.4) (layer "F.Cu") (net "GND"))
 (segment (start 74.6 115.24) (end 74.6 117.78) (width 0.4) (layer "F.Cu") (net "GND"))
 (segment (start 72.06 117.78) (end 69.52 117.78) (width 0.4) (layer "F.Cu") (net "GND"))
 (segment (start 84.76 133.02) (end 72.06 133.02) (width 0.2) (layer "F.Cu") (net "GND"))
 (segment (start 96.19 138.1) (end 84.76 138.1) (width 0.2) (layer "F.Cu") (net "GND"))
 (segment (start 107.62 107.62) (end 107.62 110.16) (width 0.4) (layer "F.Cu") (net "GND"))
 (segment (start 84.76 138.1) (end 84.76 135.56) (width 0.2) (layer "F.Cu") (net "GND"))
 (segment (start 84.76 135.56) (end 84.76 130.48) (width 0.4) (layer "F.Cu") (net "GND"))
 (segment (start 69.52 115.24) (end 69.52 110.16) (width 0.4) (layer "F.Cu") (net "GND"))
 (segment (start 125.4 107.62) (end 117.78 107.62) (width 0.4) (layer "F.Cu") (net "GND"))
 (segment (start 125.4 105.08) (end 125.4 107.62) (width 0.4) (layer "F.Cu") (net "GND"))
 (segment (start 120.32 89.84) (end 120.32 92.38) (width 0.4) (layer "F.Cu") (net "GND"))
 (segment (start 72.06 139.37) (end 72.06 135.56) (width 0.2) (layer "F.Cu") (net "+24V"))
 (segment (start 77.14 112.7) (end 77.14 115.24) (width 0.4) (layer "F.Cu") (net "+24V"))
 (segment (start 91.11 139.37) (end 72.06 139.37) (width 0.2) (layer "F.Cu") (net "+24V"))
 (segment (start 72.06 112.7) (end 77.14 112.7) (width 0.4) (layer "F.Cu") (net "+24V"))
 (segment (start 68.2818 131.7818) (end 68.2818 116.4782) (width 0.4) (layer "B.Cu") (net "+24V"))
 (segment (start 68.2818 116.4782) (end 72.06 112.7) (width 0.4) (layer "B.Cu") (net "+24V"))
 (segment (start 72.06 135.56) (end 68.2818 131.7818) (width 0.4) (layer "B.Cu") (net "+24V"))
 (segment (start 97.06 102.94) (end 123.025686 102.94) (width 0.2) (layer "B.Cu") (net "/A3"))
 (segment (start 123.025686 102.94) (end 123.425686 102.54) (width 0.2) (layer "B.Cu") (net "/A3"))
 (segment (start 123.425686 102.54) (end 125.4 102.54) (width 0.2) (layer "B.Cu") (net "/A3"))
 (segment (start 84.76 115.24) (end 97.06 102.94) (width 0.2) (layer "B.Cu") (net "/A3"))
 (segment (start 125.4 102.54) (end 138.1 89.84) (width 0.2) (layer "B.Cu") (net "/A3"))
 (segment (start 79.68 115.24) (end 84.76 115.24) (width 0.2) (layer "B.Cu") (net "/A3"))
 (segment (start 94.92 102.54) (end 122.86 102.54) (width 0.2) (layer "B.Cu") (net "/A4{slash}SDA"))
 (segment (start 84.76 112.7) (end 94.92 102.54) (width 0.2) (layer "B.Cu") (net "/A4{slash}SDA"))
 (segment (start 122.86 102.54) (end 135.56 89.84) (width 0.2) (layer "B.Cu") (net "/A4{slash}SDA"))
 (segment (start 148.26 102.54) (end 148.26 105.08) (width 0.4) (layer "F.Cu") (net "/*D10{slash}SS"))
 (segment (start 84.76 97.46) (end 87.3 97.46) (width 0.4) (layer "F.Cu") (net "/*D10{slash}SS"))
 (segment (start 87.3 97.46) (end 87.3 102.54) (width 0.4) (layer "F.Cu") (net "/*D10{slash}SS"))
 (segment (start 87.3 102.54) (end 148.26 102.54) (width 0.4) (layer "F.Cu") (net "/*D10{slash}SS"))
 (segment (start 153.34 100) (end 153.34 89.84) (width 0.4) (layer "F.Cu") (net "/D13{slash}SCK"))
 (segment (start 84.76 94.92) (end 89.84 94.92) (width 0.4) (layer "F.Cu") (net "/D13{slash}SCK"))
 (segment (start 89.84 94.92) (end 89.84 100) (width 0.4) (layer "F.Cu") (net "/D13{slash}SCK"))
 (segment (start 89.84 100) (end 153.34 100) (width 0.4) (layer "F.Cu") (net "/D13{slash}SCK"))
 (segment (start 69.52 89.84) (end 74.6 89.84) (width 0.4) (layer "F.Cu") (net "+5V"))
 (segment (start 69.52 97.46) (end 69.52 89.84) (width 0.4) (layer "F.Cu") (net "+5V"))
 (segment (start 143.18 120.32) (end 112.7 120.32) (width 0.4) (layer "F.Cu") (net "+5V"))
 (segment (start 72.06 97.46) (end 69.52 97.46) (width 0.4) (layer "F.Cu") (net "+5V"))
 (segment (start 110.16 110.16) (end 110.16 120.32) (width 0.4) (layer "F.Cu") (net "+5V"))
 (segment (start 110.16 120.32) (end 112.7 120.32) (width 0.4) (layer "F.Cu") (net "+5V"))
 (segment (start 83.775256 136.86) (end 74.6 127.684744) (width 0.2) (layer "B.Cu") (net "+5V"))
 (segment (start 72.06 120.32) (end 75.87 116.51) (width 0.2) (layer "B.Cu") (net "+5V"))
 (segment (start 85.744744 136.86) (end 83.775256 136.86) (width 0.2) (layer "B.Cu") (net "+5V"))
 (segment (start 74.6 89.84) (end 75.87 88.57) (width 0.4) (layer "B.Cu") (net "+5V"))
 (segment (start 75.87 88.57) (end 116.51 88.57) (width 0.4) (layer "B.Cu") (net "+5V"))
 (segment (start 91.11 131.494744) (end 85.744744 136.86) (width 0.2) (layer "B.Cu") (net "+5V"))
 (segment (start 119.03 88.59) (end 117.78 89.84) (width 0.4) (layer "B.Cu") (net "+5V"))
 (segment (start 125.4 89.84) (end 124.15 88.59) (width 0.4) (layer "B.Cu") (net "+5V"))
 (segment (start 124.15 88.59) (end 119.03 88.59) (width 0.4) (layer "B.Cu") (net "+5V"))
 (segment (start 75.87 101.27) (end 72.06 97.46) (width 0.2) (layer "B.Cu") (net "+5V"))
 (segment (start 74.6 127.684744) (end 74.6 122.86) (width 0.2) (layer "B.Cu") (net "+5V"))
 (segment (start 116.51 88.57) (end 117.78 89.84) (width 0.4) (layer "B.Cu") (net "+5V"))
 (segment (start 97.46 120.32) (end 112.7 120.32) (width 0.2) (layer "B.Cu") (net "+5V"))
 (segment (start 91.11 126.67) (end 97.46 120.32) (width 0.2) (layer "B.Cu") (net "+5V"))
 (segment (start 75.87 116.51) (end 75.87 101.27) (width 0.2) (layer "B.Cu") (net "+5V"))
 (segment (start 91.11 126.67) (end 91.11 131.494744) (width 0.2) (layer "B.Cu") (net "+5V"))
 (segment (start 74.6 122.86) (end 72.06 120.32) (width 0.2) (layer "B.Cu") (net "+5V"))
 (segment (start 69.52 100) (end 72.06 100) (width 0.4) (layer "F.Cu") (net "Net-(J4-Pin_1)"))
 (segment (start 69.52 102.54) (end 72.06 102.54) (width 0.4) (layer "F.Cu") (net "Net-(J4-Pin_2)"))
 (segment (start 69.52 105.08) (end 72.06 105.08) (width 0.4) (layer "F.Cu") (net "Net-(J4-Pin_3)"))
 (segment (start 69.52 107.62) (end 72.06 107.62) (width 0.4) (layer "F.Cu") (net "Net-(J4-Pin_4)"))
 (segment (start 145.72 97.46) (end 145.72 89.84) (width 0.4) (layer "F.Cu") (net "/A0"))
 (segment (start 110.16 97.46) (end 145.72 97.46) (width 0.4) (layer "F.Cu") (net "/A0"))
 (segment (start 143.18 112.7) (end 143.18 110.16) (width 0.4) (layer "F.Cu") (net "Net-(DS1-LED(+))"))
 (segment (start 112.7 112.7) (end 112.7 110.16) (width 0.4) (layer "F.Cu") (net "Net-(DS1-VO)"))
 (segment (start 115.24 117.78) (end 115.24 110.16) (width 0.4) (layer "F.Cu") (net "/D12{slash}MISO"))
 (segment (start 153.34 117.78) (end 153.34 105.08) (width 0.4) (layer "F.Cu") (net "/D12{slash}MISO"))
 (segment (start 153.34 117.78) (end 115.24 117.78) (width 0.4) (layer "F.Cu") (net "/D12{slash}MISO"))
 (segment (start 150.8 105.08) (end 150.8 115.24) (width 0.4) (layer "F.Cu") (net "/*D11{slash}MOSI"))
 (segment (start 150.8 115.24) (end 120.32 115.24) (width 0.4) (layer "F.Cu") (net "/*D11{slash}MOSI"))
 (segment (start 120.32 115.24) (end 120.32 110.16) (width 0.4) (layer "F.Cu") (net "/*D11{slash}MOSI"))
 (segment (start 133.02 105.08) (end 133.02 110.16) (width 0.4) (layer "F.Cu") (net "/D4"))
 (segment (start 135.56 110.16) (end 135.56 105.08) (width 0.4) (layer "F.Cu") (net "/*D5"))
 (segment (start 138.1 105.08) (end 138.1 110.16) (width 0.4) (layer "F.Cu") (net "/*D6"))
 (segment (start 140.64 110.16) (end 140.64 105.08) (width 0.4) (layer "F.Cu") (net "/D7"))
 (segment (start 97.46 97.46) (end 97.46 94.92) (width 0.4) (layer "F.Cu") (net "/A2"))
 (segment (start 140.64 94.92) (end 140.64 89.84) (width 0.4) (layer "F.Cu") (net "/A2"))
 (segment (start 97.46 94.92) (end 140.64 94.92) (width 0.4) (layer "F.Cu") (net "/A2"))
 (segment (start 122.86 101.27) (end 127.94 101.27) (width 0.2) (layer "F.Cu") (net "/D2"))
 (via (at 122.86 101.27) (size 0.6) (drill 0.4) (layers "F.Cu" "B.Cu") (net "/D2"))
 (via (at 127.94 101.27) (size 0.6) (drill 0.4) (layers "F.Cu" "B.Cu") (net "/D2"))
 (segment (start 79.68 89.84) (end 82.25 92.41) (width 0.2) (layer "B.Cu") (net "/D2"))
 (segment (start 87.33 92.41) (end 91.11 96.19) (width 0.2) (layer "B.Cu") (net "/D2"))
 (segment (start 117.78 96.19) (end 122.86 101.27) (width 0.2) (layer "B.Cu") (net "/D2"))
 (segment (start 82.25 92.41) (end 87.33 92.41) (width 0.2) (layer "B.Cu") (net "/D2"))
 (segment (start 91.11 96.19) (end 117.78 96.19) (width 0.2) (layer "B.Cu") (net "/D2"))
 (segment (start 127.94 101.27) (end 127.94 105.08) (width 0.2) (layer "B.Cu") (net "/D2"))
 (segment (start 130.48 98.73) (end 125.4 98.73) (width 0.2) (layer "F.Cu") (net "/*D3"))
 (via (at 125.4 98.73) (size 0.6) (drill 0.4) (layers "F.Cu" "B.Cu") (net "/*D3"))
 (via (at 130.48 98.73) (size 0.6) (drill 0.4) (layers "F.Cu" "B.Cu") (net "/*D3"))
 (segment (start 88.57 89.84) (end 82.22 89.84) (width 0.2) (layer "B.Cu") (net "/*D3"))
 (segment (start 92.38 93.65) (end 88.57 89.84) (width 0.2) (layer "B.Cu") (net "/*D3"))
 (segment (start 120.32 93.65) (end 92.38 93.65) (width 0.2) (layer "B.Cu") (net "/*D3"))
 (segment (start 130.48 105.08) (end 130.48 98.73) (width 0.2) (layer "B.Cu") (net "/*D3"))
 (segment (start 125.4 98.73) (end 120.32 93.65) (width 0.2) (layer "B.Cu") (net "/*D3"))
 (segment (start 84.221522 116.48) (end 84.191522 116.51) (width 0.2) (layer "B.Cu") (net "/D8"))
 (segment (start 85.298478 116.48) (end 84.221522 116.48) (width 0.2) (layer "B.Cu") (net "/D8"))
 (segment (start 84.191522 116.51) (end 83.49 116.51) (width 0.2) (layer "B.Cu") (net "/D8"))
 (segment (start 83.49 116.51) (end 82.22 117.78) (width 0.2) (layer "B.Cu") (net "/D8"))
 (segment (start 82.22 119.05) (end 83.49 120.32) (width 0.2) (layer "B.Cu") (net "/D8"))
 (segment (start 82.22 117.78) (end 82.22 119.05) (width 0.2) (layer "B.Cu") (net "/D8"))
 (segment (start 86.734314 116.51) (end 85.328478 116.51) (width 0.2) (layer "B.Cu") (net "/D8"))
 (segment (start 96.024314 107.22) (end 86.734314 116.51) (width 0.2) (layer "B.Cu") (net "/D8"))
 (segment (start 83.49 120.32) (end 84.76 120.32) (width 0.2) (layer "B.Cu") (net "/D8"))
 (segment (start 143.18 105.08) (end 141.04 107.22) (width 0.2) (layer "B.Cu") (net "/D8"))
 (segment (start 85.328478 116.51) (end 85.298478 116.48) (width 0.2) (layer "B.Cu") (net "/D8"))
 (segment (start 141.04 107.22) (end 96.024314 107.22) (width 0.2) (layer "B.Cu") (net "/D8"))
 (segment (start 84.76 117.78) (end 86.03 117.78) (width 0.2) (layer "B.Cu") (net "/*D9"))
 (segment (start 143.18 107.62) (end 145.72 105.08) (width 0.2) (layer "B.Cu") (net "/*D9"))
 (segment (start 86.03 117.78) (end 96.19 107.62) (width 0.2) (layer "B.Cu") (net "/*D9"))
 (segment (start 96.19 107.62) (end 143.18 107.62) (width 0.2) (layer "B.Cu") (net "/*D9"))
 (segment (start 69.52 122.86) (end 72.06 122.86) (width 0.4) (layer "F.Cu") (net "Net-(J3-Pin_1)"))
 (segment (start 69.52 125.4) (end 72.06 125.4) (width 0.4) (layer "F.Cu") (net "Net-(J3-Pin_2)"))
 (segment (start 69.52 127.94) (end 72.06 127.94) (width 0.4) (layer "F.Cu") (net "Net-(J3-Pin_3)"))
 (segment (start 69.52 130.48) (end 72.06 130.48) (width 0.4) (layer "F.Cu") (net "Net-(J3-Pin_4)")))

